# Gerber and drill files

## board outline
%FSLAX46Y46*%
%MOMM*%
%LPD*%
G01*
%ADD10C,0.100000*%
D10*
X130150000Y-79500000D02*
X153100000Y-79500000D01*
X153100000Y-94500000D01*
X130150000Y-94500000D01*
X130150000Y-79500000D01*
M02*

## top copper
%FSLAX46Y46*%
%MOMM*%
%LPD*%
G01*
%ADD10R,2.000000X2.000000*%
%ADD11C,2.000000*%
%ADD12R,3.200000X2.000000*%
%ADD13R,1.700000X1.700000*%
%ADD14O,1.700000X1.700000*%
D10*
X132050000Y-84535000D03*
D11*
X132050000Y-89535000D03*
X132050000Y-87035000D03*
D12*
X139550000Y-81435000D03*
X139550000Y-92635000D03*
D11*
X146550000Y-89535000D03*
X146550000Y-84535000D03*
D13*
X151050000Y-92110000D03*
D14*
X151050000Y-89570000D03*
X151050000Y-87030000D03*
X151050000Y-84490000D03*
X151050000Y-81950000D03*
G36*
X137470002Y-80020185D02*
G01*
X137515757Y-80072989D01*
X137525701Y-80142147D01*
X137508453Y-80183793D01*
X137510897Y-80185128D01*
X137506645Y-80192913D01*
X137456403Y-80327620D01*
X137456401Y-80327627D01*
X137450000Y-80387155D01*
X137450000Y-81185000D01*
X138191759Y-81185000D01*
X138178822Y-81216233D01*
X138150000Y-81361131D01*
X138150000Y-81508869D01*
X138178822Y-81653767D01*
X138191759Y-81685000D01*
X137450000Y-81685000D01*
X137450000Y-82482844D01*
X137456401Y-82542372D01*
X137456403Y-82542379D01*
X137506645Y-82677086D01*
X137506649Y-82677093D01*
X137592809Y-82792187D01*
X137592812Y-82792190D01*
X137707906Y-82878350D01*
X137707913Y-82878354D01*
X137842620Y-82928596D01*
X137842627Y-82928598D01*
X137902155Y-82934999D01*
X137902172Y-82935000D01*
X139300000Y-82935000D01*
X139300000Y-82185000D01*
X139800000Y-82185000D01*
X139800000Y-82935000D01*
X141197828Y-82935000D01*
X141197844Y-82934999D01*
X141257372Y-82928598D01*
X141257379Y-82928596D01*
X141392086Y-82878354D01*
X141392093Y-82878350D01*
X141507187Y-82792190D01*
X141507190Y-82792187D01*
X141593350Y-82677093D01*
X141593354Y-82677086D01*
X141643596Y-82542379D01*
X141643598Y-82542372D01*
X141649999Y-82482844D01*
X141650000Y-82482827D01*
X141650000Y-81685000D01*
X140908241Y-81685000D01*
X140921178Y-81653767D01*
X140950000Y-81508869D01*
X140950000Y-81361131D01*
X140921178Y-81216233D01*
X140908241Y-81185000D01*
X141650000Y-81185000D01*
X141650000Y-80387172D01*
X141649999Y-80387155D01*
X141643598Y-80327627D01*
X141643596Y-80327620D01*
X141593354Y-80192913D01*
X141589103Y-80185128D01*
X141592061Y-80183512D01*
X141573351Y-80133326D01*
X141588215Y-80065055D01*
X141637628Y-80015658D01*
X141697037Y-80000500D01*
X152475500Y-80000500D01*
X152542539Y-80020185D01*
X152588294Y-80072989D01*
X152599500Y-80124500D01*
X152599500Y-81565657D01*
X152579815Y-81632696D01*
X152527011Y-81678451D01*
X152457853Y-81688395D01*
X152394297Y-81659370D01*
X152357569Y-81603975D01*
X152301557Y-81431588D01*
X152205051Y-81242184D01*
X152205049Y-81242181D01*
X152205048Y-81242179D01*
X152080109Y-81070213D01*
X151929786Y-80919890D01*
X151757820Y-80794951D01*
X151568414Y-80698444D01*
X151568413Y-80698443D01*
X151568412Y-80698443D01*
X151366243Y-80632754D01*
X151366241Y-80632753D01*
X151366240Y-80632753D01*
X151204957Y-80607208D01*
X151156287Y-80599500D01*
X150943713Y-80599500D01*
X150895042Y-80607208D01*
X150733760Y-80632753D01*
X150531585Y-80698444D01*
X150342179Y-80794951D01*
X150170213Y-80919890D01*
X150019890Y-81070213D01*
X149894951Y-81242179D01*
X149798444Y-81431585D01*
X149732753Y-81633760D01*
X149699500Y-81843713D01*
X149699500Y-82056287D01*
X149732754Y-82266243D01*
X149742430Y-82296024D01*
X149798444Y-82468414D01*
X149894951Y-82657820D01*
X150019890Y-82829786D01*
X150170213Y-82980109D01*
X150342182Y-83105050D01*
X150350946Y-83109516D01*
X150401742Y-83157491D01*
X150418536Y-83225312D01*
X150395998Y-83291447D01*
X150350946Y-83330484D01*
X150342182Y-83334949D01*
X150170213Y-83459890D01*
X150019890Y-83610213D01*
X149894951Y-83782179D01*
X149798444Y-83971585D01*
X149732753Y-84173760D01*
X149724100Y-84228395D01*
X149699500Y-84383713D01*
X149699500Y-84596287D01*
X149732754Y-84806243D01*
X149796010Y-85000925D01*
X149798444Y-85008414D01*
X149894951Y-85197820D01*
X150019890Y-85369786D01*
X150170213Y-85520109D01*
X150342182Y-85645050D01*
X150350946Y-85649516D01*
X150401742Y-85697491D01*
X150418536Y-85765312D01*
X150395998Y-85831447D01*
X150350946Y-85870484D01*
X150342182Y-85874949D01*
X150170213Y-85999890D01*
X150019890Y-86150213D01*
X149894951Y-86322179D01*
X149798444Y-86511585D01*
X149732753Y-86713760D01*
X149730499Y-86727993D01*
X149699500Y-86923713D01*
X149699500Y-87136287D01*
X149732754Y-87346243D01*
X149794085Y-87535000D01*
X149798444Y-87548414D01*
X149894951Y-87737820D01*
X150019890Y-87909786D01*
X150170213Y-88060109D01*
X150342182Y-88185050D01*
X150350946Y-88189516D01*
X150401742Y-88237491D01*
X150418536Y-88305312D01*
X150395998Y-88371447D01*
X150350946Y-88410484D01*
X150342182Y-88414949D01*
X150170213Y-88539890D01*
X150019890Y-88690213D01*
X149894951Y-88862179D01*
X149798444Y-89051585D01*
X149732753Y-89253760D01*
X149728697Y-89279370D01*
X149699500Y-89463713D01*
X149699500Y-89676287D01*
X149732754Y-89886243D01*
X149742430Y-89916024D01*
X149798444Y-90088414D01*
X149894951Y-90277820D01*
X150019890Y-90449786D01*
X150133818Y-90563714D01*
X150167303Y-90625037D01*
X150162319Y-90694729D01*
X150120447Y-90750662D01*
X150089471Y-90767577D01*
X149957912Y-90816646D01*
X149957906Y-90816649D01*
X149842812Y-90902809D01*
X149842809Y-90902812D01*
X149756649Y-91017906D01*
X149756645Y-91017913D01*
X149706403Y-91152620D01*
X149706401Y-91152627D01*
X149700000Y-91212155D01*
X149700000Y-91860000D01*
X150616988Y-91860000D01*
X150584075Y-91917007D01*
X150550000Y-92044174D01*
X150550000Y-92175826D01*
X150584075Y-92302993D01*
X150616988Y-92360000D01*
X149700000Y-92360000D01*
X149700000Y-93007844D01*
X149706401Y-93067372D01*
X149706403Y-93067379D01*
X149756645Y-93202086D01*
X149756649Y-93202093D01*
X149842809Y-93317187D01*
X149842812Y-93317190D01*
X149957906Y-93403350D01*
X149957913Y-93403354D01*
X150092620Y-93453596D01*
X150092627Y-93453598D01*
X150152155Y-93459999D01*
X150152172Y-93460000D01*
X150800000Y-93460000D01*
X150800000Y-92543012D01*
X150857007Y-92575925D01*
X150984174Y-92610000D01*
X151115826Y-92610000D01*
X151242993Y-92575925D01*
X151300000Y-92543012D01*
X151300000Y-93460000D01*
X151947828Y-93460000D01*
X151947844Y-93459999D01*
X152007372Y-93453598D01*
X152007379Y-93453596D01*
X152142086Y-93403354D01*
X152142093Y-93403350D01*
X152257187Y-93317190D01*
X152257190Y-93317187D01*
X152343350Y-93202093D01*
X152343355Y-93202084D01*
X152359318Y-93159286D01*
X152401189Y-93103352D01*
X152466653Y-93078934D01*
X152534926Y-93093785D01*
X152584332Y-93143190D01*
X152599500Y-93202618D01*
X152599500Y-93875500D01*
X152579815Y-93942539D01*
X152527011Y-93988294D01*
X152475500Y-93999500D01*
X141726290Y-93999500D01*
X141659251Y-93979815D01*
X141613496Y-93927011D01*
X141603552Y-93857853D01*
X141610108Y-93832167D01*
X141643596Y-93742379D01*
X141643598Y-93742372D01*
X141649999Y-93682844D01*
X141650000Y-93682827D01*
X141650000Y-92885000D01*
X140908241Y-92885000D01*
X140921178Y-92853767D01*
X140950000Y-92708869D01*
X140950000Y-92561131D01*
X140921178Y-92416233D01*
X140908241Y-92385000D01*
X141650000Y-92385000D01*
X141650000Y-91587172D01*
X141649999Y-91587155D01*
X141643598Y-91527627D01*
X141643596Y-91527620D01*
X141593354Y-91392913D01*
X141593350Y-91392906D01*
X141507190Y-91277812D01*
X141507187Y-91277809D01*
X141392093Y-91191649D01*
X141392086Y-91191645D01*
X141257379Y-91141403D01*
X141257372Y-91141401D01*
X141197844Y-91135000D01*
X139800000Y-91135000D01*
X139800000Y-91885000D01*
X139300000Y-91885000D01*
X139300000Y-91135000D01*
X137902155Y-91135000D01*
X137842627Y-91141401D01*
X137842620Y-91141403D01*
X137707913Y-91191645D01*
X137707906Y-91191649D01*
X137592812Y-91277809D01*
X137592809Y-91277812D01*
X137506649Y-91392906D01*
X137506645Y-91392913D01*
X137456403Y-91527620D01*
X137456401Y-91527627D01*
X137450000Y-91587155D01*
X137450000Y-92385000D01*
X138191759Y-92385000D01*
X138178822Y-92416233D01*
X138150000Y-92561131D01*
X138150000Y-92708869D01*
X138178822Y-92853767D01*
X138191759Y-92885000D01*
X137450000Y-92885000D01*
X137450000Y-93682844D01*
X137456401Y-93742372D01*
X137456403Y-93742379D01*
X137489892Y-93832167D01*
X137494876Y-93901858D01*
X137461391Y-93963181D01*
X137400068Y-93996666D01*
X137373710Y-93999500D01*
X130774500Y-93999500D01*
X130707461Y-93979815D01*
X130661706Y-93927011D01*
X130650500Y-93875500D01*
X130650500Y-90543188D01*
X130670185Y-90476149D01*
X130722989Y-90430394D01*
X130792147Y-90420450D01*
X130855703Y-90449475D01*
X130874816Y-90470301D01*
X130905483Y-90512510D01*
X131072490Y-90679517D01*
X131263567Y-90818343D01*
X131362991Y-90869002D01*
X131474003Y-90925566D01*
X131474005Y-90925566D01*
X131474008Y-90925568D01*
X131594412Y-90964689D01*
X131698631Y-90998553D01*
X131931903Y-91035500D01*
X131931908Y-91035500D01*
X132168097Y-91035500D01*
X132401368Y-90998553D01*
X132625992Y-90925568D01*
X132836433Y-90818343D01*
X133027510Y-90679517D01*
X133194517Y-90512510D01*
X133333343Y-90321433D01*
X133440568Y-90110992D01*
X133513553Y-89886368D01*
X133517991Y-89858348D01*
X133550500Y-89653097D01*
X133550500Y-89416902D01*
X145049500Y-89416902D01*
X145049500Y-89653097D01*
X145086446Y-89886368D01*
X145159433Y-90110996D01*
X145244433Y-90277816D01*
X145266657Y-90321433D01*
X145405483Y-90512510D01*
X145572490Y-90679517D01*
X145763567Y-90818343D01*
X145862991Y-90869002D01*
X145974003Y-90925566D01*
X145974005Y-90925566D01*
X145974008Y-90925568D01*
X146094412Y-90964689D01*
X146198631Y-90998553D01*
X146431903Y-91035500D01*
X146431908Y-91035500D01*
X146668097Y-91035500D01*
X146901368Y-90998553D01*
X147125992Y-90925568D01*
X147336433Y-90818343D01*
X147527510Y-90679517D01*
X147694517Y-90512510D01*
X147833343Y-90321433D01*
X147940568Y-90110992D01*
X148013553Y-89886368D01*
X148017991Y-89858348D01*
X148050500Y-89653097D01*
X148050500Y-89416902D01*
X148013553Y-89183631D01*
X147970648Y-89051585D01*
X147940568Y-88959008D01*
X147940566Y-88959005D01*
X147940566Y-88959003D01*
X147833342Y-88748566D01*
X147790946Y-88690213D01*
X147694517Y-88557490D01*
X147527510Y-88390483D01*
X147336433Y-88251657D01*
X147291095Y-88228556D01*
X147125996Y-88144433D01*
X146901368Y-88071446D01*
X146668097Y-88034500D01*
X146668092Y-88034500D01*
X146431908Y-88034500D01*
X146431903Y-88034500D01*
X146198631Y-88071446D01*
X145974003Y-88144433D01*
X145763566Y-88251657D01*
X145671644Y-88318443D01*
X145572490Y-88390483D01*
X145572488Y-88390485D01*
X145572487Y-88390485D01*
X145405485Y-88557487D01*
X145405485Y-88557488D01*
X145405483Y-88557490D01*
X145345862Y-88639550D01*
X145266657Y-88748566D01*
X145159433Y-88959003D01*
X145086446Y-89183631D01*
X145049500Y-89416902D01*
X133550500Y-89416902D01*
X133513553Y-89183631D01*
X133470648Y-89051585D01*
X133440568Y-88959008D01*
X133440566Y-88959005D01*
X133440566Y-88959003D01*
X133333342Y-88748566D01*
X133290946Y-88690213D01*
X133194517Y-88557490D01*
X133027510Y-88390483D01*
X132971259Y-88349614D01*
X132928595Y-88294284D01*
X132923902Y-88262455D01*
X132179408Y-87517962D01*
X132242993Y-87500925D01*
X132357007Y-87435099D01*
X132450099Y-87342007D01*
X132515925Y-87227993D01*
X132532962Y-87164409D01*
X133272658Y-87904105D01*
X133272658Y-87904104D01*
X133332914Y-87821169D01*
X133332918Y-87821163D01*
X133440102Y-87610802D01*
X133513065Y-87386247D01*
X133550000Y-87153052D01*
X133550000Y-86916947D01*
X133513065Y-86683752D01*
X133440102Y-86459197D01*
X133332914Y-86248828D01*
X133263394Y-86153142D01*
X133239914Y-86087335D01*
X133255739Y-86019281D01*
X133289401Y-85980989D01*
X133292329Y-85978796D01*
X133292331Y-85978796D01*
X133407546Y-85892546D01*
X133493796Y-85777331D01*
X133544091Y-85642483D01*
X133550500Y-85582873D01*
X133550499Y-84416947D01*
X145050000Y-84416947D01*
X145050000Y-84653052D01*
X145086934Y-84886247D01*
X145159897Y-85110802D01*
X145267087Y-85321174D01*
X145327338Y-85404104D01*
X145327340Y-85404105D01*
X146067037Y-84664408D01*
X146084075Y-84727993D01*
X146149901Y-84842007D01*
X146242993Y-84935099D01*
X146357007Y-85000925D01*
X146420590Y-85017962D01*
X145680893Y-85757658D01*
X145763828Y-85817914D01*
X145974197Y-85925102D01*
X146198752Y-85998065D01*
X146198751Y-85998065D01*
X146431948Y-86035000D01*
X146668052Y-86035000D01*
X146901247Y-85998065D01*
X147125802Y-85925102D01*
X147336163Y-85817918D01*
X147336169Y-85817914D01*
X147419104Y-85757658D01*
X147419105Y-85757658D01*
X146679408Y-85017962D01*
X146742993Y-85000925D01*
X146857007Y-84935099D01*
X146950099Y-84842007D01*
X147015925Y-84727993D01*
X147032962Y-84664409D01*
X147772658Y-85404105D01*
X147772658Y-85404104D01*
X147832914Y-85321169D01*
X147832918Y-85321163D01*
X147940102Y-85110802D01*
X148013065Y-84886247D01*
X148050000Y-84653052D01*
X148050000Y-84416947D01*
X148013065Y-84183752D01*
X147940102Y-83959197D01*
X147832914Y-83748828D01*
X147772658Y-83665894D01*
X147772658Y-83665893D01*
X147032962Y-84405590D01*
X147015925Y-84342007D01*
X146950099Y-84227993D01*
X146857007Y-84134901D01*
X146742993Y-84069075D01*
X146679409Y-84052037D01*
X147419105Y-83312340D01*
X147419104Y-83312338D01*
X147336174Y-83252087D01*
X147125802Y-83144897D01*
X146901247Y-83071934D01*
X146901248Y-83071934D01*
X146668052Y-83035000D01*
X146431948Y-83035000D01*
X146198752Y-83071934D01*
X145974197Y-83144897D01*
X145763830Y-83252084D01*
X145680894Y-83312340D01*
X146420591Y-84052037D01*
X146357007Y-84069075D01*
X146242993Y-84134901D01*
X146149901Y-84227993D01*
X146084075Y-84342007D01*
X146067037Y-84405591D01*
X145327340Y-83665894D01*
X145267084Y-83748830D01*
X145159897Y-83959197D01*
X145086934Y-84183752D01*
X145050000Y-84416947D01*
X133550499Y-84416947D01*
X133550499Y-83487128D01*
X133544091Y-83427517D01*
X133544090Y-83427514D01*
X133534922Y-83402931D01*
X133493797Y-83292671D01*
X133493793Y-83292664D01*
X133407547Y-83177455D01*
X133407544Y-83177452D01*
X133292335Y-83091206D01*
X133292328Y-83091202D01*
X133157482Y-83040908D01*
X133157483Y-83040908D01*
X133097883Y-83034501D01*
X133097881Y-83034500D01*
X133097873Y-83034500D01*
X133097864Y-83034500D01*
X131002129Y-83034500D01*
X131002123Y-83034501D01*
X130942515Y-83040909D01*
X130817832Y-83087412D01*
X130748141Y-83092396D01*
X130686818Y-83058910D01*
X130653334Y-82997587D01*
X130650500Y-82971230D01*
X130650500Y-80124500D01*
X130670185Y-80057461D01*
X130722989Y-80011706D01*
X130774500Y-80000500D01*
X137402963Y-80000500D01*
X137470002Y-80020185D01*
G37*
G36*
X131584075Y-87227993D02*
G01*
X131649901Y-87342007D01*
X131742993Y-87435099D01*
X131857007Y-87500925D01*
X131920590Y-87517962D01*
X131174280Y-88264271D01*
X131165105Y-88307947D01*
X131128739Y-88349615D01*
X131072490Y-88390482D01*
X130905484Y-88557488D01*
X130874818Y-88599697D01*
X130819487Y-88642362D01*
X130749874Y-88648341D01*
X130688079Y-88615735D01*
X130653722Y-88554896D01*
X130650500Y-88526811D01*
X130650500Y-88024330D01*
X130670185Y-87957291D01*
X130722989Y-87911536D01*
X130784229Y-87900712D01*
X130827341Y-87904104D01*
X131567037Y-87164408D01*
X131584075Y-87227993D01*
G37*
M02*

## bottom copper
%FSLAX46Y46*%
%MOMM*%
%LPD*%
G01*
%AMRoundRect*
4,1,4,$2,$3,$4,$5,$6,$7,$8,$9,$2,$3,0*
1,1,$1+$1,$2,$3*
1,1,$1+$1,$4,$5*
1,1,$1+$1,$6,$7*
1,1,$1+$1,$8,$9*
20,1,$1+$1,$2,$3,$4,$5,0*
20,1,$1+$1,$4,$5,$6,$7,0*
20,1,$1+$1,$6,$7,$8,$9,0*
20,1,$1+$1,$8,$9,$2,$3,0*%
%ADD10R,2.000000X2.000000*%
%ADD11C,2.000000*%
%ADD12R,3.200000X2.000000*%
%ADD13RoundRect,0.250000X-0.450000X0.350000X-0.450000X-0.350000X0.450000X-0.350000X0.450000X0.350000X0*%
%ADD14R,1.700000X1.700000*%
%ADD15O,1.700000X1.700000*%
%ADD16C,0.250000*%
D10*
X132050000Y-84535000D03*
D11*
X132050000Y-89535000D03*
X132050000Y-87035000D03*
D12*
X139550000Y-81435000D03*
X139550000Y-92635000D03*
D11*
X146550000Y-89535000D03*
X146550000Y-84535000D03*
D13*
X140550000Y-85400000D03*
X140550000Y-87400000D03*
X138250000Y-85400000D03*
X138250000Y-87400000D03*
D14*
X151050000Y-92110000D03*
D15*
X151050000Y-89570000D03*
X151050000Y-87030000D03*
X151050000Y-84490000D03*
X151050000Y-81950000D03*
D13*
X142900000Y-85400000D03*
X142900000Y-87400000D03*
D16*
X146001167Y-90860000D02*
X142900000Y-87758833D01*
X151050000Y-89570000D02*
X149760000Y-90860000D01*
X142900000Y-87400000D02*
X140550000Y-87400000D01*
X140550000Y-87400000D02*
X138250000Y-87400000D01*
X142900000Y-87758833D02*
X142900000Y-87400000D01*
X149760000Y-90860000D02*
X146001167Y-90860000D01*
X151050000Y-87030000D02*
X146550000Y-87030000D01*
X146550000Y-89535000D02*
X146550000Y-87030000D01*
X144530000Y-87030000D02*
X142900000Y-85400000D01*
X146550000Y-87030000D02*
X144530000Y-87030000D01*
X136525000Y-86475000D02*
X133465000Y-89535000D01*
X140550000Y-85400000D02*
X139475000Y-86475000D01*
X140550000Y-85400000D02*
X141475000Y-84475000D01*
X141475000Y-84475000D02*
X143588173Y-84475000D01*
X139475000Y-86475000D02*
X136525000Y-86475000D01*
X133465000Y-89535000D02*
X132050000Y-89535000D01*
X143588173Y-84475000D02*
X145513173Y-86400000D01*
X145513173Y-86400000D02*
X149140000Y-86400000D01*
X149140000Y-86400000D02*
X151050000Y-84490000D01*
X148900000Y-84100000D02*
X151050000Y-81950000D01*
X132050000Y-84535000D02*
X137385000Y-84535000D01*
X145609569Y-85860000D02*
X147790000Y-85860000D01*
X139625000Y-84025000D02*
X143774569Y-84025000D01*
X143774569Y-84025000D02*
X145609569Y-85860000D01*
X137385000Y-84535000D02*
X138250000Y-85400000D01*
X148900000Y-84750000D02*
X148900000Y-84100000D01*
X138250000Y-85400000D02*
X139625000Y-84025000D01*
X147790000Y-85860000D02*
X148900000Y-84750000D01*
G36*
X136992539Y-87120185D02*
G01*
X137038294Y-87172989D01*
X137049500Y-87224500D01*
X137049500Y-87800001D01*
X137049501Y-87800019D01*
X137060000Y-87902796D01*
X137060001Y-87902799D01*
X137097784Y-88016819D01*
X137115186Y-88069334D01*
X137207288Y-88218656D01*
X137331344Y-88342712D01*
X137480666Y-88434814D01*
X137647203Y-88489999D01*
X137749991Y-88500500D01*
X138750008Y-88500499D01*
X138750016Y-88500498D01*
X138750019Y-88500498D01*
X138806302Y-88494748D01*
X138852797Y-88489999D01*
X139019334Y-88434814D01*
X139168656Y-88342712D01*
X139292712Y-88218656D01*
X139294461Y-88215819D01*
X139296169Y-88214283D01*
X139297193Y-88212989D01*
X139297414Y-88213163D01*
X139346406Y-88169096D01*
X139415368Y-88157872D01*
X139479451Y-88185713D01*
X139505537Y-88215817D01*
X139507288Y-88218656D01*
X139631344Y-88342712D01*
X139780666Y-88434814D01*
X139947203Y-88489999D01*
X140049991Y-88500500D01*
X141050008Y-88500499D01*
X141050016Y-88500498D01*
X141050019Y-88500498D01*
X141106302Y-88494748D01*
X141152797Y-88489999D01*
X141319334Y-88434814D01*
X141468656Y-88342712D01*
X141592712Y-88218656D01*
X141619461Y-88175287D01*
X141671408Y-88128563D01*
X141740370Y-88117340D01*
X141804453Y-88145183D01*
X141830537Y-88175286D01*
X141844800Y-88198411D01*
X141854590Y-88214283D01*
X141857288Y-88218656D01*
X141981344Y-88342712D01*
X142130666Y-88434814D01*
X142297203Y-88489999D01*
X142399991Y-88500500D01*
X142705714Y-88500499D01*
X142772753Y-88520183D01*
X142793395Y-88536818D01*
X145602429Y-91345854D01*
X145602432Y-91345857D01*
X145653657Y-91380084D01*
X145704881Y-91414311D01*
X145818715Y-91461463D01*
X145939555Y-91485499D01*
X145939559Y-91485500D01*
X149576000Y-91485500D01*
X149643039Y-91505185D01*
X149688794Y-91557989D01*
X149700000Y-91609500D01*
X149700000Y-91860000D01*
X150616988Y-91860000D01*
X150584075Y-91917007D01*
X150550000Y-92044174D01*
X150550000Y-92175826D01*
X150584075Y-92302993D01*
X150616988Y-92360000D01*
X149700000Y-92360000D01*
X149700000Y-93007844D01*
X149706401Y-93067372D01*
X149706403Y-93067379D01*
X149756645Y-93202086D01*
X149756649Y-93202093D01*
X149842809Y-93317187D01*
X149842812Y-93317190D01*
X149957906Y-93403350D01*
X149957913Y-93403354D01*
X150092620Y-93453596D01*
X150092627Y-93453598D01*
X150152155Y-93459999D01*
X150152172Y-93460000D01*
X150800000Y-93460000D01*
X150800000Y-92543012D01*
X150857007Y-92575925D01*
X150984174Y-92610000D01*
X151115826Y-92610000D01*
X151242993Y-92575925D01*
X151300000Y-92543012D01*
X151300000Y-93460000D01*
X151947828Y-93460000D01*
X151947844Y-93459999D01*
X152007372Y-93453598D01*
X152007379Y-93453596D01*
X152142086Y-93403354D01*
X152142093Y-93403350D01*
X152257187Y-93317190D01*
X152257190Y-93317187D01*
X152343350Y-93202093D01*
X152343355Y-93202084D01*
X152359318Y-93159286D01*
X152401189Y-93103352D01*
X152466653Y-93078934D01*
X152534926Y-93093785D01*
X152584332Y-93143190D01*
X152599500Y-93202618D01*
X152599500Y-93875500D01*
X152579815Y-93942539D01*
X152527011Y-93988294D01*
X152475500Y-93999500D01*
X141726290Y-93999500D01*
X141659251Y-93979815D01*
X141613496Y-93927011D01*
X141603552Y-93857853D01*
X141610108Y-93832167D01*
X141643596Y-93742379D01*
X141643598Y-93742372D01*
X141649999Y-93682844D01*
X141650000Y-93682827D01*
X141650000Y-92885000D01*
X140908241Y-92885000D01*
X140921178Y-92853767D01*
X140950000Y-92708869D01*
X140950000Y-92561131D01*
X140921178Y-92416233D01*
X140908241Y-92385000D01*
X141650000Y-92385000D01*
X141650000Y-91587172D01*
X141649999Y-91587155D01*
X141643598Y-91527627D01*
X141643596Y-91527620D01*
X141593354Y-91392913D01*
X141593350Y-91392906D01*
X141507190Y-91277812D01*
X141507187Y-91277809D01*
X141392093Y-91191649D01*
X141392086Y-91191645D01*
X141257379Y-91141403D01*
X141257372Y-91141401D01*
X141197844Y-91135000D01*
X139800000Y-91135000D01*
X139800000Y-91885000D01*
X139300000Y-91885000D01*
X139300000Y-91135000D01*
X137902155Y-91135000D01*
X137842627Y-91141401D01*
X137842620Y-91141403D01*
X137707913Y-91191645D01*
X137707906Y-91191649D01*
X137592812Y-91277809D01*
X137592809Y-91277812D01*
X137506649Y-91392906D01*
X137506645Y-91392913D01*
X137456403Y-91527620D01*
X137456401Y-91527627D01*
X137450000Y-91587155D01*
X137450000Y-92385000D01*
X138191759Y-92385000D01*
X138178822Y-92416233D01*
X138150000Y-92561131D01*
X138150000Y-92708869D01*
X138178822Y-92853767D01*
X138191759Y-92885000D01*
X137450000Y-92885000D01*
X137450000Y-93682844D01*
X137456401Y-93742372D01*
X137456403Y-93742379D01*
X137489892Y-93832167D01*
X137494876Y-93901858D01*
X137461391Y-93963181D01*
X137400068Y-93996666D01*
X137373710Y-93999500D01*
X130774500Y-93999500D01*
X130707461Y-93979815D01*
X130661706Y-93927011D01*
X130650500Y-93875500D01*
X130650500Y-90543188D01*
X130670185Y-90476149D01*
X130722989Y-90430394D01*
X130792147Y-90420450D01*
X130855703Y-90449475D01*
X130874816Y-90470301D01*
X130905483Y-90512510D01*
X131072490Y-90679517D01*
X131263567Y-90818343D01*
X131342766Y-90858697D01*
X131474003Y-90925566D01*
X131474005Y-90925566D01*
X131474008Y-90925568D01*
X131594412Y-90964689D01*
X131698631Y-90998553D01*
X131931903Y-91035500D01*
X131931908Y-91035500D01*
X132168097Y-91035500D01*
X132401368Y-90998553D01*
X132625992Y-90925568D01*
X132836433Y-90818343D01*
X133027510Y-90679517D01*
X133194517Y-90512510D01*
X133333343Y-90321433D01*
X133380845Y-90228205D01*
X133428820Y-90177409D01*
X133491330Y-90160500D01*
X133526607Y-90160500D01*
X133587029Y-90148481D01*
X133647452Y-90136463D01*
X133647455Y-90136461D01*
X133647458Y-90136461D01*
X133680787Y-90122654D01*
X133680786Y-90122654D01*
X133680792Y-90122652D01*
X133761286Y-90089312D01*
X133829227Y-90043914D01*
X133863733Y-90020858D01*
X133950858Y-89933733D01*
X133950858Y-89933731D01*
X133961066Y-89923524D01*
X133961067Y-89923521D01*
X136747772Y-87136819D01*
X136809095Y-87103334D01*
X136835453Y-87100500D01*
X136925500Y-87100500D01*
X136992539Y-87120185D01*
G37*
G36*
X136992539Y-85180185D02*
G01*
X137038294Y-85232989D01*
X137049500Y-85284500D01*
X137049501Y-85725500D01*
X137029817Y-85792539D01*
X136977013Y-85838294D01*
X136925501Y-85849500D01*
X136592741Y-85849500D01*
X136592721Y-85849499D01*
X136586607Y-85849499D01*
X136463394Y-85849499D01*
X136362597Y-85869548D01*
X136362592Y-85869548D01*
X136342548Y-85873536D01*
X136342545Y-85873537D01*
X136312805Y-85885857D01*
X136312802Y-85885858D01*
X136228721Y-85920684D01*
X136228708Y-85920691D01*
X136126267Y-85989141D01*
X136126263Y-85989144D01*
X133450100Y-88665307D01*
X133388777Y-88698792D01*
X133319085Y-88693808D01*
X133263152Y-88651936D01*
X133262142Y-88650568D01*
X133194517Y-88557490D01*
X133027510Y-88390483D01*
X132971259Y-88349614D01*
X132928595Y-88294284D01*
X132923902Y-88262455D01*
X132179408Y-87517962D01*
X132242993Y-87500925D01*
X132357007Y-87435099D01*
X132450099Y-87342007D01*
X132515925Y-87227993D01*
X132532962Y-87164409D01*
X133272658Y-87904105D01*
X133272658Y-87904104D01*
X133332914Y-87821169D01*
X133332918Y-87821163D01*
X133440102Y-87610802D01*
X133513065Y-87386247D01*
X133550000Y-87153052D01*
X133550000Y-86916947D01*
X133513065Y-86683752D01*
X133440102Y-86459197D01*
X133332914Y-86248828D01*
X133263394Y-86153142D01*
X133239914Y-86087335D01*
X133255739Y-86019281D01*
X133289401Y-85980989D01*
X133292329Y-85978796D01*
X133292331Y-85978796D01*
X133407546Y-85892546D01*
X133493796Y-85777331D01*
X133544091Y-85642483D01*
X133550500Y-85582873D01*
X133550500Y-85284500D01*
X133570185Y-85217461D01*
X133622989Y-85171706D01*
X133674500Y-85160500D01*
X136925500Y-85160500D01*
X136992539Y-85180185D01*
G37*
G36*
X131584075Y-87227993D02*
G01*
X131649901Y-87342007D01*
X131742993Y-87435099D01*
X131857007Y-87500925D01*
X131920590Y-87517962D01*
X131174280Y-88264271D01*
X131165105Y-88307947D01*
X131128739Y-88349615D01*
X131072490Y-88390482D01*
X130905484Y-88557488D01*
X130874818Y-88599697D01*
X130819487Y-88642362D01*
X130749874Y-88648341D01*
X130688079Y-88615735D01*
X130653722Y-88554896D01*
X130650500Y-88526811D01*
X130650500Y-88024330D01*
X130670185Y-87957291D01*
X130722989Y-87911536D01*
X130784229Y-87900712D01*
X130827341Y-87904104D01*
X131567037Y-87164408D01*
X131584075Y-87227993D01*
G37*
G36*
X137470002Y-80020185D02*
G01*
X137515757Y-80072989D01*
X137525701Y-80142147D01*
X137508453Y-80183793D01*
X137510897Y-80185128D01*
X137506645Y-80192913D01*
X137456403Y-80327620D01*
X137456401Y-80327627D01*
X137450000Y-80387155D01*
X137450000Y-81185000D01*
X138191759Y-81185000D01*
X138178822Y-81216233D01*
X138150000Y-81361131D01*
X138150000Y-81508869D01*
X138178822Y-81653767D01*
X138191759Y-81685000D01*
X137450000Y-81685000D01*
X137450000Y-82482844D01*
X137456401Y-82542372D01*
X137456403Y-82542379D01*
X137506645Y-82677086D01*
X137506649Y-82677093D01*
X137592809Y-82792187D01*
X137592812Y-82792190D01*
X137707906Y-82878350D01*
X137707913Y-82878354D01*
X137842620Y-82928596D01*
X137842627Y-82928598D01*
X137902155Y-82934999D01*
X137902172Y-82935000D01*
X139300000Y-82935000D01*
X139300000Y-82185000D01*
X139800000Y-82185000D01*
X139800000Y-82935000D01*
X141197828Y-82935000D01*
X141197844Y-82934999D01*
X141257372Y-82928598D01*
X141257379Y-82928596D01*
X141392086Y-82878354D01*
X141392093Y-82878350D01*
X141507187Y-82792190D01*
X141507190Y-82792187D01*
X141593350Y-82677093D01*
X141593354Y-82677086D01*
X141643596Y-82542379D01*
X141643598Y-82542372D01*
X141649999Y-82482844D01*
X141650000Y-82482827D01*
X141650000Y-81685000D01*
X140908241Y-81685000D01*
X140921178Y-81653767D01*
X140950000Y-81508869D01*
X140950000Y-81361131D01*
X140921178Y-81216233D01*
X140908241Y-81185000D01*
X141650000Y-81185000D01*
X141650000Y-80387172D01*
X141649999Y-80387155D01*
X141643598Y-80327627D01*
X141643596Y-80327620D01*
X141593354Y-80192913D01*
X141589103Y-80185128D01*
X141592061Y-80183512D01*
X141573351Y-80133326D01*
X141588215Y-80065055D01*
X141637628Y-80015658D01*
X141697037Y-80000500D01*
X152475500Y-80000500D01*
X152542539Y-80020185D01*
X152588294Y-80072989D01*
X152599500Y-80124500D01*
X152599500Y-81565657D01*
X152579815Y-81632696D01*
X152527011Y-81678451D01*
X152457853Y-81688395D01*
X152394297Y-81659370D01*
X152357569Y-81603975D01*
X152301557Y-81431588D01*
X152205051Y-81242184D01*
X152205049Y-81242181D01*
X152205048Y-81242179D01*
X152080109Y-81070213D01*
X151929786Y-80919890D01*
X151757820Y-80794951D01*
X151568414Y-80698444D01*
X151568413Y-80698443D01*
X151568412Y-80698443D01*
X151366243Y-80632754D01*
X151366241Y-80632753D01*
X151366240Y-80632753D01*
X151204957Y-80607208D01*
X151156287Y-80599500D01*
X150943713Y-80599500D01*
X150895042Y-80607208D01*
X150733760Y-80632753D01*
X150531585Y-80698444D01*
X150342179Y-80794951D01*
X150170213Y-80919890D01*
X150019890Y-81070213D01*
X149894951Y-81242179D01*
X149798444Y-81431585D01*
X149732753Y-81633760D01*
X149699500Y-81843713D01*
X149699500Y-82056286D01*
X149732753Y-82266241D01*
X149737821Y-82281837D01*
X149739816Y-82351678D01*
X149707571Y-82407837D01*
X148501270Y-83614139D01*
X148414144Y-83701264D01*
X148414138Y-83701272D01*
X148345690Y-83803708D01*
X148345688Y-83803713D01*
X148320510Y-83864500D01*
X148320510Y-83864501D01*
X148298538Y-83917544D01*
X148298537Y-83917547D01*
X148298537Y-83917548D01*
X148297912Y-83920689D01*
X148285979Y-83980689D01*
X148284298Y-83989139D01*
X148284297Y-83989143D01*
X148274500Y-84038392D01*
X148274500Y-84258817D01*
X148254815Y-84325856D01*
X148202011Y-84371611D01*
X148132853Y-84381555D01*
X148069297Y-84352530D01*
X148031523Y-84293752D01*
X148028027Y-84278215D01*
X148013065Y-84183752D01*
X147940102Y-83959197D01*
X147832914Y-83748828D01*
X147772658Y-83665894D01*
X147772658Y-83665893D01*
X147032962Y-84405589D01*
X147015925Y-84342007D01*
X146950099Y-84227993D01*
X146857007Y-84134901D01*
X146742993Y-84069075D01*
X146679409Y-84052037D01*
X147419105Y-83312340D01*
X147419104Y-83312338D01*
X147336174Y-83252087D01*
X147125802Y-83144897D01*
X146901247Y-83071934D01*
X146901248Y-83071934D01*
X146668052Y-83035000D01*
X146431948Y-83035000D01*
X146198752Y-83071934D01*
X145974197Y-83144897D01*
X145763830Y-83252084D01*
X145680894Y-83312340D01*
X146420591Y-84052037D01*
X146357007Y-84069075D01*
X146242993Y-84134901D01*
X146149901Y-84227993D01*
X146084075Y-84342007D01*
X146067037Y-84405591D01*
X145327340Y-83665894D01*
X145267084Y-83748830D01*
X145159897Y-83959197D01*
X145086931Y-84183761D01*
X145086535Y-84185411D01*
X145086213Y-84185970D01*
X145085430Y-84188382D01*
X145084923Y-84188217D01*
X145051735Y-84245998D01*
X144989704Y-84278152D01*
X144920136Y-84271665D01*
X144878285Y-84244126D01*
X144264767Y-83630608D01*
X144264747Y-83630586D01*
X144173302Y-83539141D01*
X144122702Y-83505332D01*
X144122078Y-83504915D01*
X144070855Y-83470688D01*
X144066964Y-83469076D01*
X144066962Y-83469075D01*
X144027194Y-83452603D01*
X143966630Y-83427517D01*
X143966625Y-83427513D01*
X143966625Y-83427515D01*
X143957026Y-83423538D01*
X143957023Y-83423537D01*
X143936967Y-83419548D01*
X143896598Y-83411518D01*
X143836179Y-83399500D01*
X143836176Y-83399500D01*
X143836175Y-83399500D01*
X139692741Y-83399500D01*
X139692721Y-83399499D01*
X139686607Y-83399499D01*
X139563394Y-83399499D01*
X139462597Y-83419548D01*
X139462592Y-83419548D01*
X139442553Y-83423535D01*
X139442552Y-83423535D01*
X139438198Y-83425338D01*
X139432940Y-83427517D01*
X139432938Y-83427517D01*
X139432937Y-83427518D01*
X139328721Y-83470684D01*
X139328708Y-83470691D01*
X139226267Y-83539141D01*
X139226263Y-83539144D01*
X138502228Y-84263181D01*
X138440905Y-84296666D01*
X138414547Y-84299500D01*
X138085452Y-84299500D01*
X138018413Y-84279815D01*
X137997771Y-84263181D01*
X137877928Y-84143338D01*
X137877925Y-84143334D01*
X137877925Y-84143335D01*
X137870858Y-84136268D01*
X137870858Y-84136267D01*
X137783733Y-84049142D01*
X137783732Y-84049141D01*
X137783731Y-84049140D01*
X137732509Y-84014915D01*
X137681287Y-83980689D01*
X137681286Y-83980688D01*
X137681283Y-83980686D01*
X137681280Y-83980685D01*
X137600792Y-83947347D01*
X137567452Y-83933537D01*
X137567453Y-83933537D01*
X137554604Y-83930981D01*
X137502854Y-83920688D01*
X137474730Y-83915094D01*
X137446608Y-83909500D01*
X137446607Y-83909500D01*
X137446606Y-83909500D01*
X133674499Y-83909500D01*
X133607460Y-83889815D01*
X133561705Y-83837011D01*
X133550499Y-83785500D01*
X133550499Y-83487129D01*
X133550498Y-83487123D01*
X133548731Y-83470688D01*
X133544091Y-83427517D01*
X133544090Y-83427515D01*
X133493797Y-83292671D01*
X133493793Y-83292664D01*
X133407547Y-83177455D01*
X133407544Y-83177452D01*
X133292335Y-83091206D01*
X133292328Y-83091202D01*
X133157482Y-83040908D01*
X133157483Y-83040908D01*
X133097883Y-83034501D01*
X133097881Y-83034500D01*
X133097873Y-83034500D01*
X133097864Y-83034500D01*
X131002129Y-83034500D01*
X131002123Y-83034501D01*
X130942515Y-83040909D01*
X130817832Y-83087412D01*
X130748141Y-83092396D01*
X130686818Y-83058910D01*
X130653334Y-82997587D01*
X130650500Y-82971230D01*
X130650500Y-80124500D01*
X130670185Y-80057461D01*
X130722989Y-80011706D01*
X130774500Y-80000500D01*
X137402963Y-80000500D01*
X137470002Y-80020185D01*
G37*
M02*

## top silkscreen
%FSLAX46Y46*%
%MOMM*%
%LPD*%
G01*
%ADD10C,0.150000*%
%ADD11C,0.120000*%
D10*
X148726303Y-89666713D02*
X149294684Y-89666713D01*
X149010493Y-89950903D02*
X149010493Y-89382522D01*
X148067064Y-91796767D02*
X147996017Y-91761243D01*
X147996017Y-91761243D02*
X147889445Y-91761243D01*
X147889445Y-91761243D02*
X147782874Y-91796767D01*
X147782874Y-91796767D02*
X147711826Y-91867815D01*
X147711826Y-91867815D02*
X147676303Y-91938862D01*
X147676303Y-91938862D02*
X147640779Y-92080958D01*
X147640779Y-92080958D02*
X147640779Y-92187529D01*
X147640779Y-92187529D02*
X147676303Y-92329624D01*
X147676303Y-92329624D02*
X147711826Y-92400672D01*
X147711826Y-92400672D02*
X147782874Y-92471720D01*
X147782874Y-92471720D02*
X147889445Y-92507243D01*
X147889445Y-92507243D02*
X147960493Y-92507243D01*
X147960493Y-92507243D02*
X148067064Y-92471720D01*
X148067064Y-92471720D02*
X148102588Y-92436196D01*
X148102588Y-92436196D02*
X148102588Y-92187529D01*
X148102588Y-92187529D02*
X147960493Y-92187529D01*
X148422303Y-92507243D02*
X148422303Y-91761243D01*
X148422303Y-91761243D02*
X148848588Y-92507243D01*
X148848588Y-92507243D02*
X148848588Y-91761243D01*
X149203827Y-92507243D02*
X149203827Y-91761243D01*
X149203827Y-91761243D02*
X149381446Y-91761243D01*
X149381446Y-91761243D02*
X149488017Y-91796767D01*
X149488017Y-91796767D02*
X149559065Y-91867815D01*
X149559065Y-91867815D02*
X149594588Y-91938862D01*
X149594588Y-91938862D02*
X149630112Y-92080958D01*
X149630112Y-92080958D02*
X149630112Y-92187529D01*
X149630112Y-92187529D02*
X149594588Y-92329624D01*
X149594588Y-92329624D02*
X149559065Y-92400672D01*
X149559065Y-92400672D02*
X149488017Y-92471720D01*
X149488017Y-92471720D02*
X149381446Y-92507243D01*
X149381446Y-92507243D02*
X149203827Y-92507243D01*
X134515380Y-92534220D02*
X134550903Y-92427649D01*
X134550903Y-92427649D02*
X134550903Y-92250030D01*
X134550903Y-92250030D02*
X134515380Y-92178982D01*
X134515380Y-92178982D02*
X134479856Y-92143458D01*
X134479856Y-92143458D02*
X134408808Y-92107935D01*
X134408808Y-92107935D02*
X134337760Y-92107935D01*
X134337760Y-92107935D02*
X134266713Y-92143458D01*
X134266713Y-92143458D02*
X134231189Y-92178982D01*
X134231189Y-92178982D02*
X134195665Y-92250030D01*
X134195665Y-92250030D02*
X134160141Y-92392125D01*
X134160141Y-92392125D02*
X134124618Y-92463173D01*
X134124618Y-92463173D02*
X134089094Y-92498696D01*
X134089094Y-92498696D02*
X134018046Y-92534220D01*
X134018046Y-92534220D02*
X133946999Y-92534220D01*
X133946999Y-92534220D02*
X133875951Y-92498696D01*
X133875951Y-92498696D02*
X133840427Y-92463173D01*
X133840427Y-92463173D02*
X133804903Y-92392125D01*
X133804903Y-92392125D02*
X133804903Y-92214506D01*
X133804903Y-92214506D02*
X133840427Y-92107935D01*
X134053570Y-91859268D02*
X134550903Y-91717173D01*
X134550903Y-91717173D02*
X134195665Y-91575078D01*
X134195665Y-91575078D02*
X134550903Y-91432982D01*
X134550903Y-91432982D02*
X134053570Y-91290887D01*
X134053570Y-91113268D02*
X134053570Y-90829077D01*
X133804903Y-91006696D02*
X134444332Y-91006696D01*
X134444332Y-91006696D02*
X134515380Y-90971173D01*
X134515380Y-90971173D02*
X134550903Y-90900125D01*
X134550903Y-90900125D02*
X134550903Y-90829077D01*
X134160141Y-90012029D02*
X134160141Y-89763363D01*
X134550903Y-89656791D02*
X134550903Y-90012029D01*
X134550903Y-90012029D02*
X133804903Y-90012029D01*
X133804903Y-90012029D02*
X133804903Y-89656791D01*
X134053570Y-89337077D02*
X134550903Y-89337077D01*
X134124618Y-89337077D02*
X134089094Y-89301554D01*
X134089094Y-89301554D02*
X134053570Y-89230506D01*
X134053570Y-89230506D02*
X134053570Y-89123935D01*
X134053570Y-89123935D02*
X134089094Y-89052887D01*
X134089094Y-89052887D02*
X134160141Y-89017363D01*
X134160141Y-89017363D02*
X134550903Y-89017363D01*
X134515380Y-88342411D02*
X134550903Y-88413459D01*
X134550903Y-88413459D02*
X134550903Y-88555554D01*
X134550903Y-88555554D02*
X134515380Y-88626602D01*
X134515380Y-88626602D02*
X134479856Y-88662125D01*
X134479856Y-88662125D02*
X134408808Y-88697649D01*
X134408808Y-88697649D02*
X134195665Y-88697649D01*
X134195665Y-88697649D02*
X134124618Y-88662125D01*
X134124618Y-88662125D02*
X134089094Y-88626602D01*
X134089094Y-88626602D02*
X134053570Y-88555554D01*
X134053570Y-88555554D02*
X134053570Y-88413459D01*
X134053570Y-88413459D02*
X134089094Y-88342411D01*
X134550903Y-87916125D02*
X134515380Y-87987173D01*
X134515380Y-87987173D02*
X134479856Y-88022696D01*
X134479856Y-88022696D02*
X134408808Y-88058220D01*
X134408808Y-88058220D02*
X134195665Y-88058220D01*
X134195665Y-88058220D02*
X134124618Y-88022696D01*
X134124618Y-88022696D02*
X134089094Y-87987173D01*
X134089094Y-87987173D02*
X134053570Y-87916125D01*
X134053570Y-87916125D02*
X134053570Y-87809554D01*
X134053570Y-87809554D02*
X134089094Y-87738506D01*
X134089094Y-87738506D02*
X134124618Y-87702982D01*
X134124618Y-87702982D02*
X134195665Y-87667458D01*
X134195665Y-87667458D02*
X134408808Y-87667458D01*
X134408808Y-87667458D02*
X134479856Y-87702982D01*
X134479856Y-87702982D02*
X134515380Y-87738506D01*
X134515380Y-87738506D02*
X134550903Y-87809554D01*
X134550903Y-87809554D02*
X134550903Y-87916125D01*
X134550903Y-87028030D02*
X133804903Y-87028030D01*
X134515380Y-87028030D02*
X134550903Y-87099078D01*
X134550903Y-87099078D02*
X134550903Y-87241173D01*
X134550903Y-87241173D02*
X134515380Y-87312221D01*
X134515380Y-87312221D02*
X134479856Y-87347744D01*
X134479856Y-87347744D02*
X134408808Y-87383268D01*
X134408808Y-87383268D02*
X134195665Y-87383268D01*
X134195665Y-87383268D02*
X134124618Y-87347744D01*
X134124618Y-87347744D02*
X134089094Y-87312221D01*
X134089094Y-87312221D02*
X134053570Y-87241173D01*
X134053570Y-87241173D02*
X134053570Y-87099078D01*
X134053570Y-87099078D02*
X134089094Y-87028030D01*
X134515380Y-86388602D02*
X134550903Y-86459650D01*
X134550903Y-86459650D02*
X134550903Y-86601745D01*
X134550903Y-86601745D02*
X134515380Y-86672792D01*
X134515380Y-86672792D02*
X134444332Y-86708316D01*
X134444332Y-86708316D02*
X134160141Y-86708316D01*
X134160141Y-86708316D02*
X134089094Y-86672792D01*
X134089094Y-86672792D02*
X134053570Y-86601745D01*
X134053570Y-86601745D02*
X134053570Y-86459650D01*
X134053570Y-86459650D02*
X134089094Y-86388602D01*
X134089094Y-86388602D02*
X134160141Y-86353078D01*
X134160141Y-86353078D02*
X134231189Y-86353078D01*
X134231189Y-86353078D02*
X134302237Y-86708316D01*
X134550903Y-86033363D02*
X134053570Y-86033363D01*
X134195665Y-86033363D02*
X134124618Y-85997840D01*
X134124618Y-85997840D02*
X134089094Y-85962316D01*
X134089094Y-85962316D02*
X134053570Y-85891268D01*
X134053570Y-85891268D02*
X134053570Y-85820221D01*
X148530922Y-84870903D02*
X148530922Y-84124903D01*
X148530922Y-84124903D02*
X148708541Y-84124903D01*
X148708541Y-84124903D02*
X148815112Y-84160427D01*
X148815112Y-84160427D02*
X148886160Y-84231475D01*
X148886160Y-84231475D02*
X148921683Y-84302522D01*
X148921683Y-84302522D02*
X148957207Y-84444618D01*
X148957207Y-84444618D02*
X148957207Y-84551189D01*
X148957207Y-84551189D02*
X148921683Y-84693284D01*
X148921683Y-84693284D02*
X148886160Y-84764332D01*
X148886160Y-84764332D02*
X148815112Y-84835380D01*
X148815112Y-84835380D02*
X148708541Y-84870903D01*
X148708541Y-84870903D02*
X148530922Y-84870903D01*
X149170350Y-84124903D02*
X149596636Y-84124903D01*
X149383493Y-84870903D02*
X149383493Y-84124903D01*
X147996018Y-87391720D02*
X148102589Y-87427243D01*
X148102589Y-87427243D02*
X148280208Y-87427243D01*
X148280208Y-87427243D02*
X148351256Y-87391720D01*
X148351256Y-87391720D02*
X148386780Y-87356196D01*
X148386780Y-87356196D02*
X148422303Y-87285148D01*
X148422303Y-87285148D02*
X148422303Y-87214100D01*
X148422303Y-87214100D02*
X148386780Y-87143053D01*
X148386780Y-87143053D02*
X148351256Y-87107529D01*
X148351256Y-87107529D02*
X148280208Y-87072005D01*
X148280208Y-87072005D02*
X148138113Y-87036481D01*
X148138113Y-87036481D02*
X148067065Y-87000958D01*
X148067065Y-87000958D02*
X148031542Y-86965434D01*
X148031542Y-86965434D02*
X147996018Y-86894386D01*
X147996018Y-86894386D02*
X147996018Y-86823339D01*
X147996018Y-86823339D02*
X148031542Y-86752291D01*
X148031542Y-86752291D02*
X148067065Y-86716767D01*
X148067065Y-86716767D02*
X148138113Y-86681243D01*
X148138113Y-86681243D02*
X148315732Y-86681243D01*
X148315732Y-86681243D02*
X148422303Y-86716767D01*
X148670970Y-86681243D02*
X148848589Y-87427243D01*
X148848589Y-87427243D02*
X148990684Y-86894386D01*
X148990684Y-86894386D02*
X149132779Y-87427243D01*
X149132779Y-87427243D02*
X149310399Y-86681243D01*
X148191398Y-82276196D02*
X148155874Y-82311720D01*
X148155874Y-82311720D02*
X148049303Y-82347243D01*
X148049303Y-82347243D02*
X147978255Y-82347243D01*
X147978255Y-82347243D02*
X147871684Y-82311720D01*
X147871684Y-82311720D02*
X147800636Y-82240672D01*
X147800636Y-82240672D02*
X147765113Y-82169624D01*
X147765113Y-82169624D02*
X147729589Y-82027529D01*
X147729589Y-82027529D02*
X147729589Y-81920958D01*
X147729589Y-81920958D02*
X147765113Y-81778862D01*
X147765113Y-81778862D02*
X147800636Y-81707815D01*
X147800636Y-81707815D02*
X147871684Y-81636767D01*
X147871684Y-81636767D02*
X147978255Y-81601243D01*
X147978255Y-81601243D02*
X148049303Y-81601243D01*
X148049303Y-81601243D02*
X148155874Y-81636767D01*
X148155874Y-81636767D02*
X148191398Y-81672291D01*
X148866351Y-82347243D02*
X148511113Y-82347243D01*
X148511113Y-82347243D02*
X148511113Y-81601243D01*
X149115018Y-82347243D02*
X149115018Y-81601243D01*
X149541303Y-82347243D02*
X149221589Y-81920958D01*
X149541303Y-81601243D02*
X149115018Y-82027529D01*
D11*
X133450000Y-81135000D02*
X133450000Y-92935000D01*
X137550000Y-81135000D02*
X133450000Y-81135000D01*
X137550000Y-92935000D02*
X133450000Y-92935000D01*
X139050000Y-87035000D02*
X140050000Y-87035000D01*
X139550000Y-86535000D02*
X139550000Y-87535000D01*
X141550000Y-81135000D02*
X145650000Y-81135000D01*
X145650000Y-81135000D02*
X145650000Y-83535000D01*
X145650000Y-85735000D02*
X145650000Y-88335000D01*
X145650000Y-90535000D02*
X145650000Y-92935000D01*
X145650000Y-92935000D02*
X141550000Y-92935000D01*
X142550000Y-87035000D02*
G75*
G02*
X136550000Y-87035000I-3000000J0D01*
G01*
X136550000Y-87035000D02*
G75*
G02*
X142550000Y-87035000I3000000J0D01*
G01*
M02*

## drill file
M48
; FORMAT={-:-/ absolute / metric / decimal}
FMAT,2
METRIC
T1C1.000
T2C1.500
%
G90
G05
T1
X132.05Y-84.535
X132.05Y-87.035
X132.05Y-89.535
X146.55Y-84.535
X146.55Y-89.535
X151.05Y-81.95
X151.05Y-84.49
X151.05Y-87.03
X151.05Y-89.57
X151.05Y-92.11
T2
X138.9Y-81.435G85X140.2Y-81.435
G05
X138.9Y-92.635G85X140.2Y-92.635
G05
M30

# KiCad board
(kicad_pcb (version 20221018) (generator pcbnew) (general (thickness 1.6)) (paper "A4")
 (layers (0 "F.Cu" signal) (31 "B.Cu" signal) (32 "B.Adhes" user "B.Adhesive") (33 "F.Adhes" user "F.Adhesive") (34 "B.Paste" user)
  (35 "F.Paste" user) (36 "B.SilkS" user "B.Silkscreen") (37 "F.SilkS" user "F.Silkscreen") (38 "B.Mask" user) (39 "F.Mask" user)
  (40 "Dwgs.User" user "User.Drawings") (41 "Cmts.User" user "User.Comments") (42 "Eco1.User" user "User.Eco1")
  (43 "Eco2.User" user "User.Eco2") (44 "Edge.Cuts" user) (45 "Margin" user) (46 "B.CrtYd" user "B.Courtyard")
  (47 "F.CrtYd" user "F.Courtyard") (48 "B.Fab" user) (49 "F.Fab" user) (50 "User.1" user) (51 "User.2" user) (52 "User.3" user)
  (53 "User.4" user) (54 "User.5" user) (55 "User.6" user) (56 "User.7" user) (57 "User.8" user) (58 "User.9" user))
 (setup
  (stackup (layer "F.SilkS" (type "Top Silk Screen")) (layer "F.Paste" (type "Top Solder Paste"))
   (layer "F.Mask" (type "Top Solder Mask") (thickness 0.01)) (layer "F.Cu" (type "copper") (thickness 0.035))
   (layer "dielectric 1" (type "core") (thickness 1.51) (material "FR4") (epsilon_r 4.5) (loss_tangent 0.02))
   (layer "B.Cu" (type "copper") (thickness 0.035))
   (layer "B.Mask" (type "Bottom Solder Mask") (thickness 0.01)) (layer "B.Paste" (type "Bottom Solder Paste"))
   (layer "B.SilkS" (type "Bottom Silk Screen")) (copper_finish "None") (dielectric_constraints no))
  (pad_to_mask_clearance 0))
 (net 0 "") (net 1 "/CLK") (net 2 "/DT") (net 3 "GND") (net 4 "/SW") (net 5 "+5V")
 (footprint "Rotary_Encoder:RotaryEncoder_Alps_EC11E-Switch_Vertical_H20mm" (layer "F.Cu") (at 132.05 84.535)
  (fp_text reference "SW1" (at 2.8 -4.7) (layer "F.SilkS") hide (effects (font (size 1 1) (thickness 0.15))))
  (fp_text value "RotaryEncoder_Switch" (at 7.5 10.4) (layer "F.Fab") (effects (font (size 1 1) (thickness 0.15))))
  (fp_line (start 1.4 -3.4) (end 1.4 8.4) (stroke (width 0.12) (type solid)) (layer "F.SilkS"))
  (fp_line (start 5.5 -3.4) (end 1.4 -3.4) (stroke (width 0.12) (type solid)) (layer "F.SilkS"))
  (fp_line (start 5.5 8.4) (end 1.4 8.4) (stroke (width 0.12) (type solid)) (layer "F.SilkS"))
  (fp_line (start 7 2.5) (end 8 2.5) (stroke (width 0.12) (type solid)) (layer "F.SilkS"))
  (fp_line (start 7.5 2) (end 7.5 3) (stroke (width 0.12) (type solid)) (layer "F.SilkS"))
  (fp_line (start 9.5 -3.4) (end 13.6 -3.4) (stroke (width 0.12) (type solid)) (layer "F.SilkS"))
  (fp_line (start 13.6 -3.4) (end 13.6 -1) (stroke (width 0.12) (type solid)) (layer "F.SilkS"))
  (fp_line (start 13.6 1.2) (end 13.6 3.8) (stroke (width 0.12) (type solid)) (layer "F.SilkS"))
  (fp_line (start 13.6 6) (end 13.6 8.4) (stroke (width 0.12) (type solid)) (layer "F.SilkS"))
  (fp_line (start 13.6 8.4) (end 9.5 8.4) (stroke (width 0.12) (type solid)) (layer "F.SilkS"))
  (fp_circle (center 7.5 2.5) (end 10.5 2.5) (stroke (width 0.12) (type solid)) (fill none) (layer "F.SilkS"))
  (pad "A" thru_hole rect (at 0 0) (size 2 2) (drill 1) (layers "*.Cu" "*.Mask") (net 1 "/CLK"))
  (pad "B" thru_hole circle (at 0 5) (size 2 2) (drill 1) (layers "*.Cu" "*.Mask") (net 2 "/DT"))
  (pad "C" thru_hole circle (at 0 2.5) (size 2 2) (drill 1) (layers "*.Cu" "*.Mask") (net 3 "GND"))
  (pad "MP" thru_hole rect (at 7.5 -3.1) (size 3.2 2) (drill oval 2.8 1.5) (layers "*.Cu" "*.Mask") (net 3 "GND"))
  (pad "MP" thru_hole rect (at 7.5 8.1) (size 3.2 2) (drill oval 2.8 1.5) (layers "*.Cu" "*.Mask") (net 3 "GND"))
  (pad "S1" thru_hole circle (at 14.5 5) (size 2 2) (drill 1) (layers "*.Cu" "*.Mask") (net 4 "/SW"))
  (pad "S2" thru_hole circle (at 14.5 0) (size 2 2) (drill 1) (layers "*.Cu" "*.Mask") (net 3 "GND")))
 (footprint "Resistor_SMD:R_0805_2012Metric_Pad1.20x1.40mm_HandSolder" (layer "B.Cu") (at 140.55 86.4 -90)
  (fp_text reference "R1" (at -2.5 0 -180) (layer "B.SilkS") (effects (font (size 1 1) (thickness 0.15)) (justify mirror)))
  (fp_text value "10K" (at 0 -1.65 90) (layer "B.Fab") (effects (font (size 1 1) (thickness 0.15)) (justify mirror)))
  (pad "1" smd roundrect (at -1 0 270) (size 1.2 1.4) (layers "B.Cu" "B.Paste" "B.Mask") (roundrect_rratio 0.208333) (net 2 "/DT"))
  (pad "2" smd roundrect (at 1 0 270) (size 1.2 1.4) (layers "B.Cu" "B.Paste" "B.Mask") (roundrect_rratio 0.208333) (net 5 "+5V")))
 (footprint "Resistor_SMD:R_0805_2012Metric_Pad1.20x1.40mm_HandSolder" (layer "B.Cu") (at 138.25 86.4 -90)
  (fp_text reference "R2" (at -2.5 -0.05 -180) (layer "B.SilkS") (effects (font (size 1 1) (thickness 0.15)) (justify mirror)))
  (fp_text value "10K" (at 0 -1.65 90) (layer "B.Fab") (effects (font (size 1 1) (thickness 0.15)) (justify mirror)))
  (pad "1" smd roundrect (at -1 0 270) (size 1.2 1.4) (layers "B.Cu" "B.Paste" "B.Mask") (roundrect_rratio 0.208333) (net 1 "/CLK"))
  (pad "2" smd roundrect (at 1 0 270) (size 1.2 1.4) (layers "B.Cu" "B.Paste" "B.Mask") (roundrect_rratio 0.208333) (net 5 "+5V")))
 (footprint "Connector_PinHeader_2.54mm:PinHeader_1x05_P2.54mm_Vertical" (layer "B.Cu") (at 151.05 92.11)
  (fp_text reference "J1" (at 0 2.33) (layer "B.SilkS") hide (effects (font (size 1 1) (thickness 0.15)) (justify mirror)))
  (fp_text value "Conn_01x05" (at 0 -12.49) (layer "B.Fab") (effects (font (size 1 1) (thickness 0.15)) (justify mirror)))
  (pad "1" thru_hole rect (at 0 0) (size 1.7 1.7) (drill 1) (layers "*.Cu" "*.Mask") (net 3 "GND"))
  (pad "2" thru_hole oval (at 0 -2.54) (size 1.7 1.7) (drill 1) (layers "*.Cu" "*.Mask") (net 5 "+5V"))
  (pad "3" thru_hole oval (at 0 -5.08) (size 1.7 1.7) (drill 1) (layers "*.Cu" "*.Mask") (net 4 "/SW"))
  (pad "4" thru_hole oval (at 0 -7.62) (size 1.7 1.7) (drill 1) (layers "*.Cu" "*.Mask") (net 2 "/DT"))
  (pad "5" thru_hole oval (at 0 -10.16) (size 1.7 1.7) (drill 1) (layers "*.Cu" "*.Mask") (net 1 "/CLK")))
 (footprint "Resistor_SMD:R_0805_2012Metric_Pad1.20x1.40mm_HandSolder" (layer "B.Cu") (at 142.9 86.4 -90)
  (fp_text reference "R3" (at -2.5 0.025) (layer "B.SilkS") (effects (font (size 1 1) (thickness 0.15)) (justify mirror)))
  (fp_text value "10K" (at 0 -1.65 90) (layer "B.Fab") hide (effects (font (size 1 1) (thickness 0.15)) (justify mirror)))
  (pad "1" smd roundrect (at -1 0 270) (size 1.2 1.4) (layers "B.Cu" "B.Paste" "B.Mask") (roundrect_rratio 0.208333) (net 4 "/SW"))
  (pad "2" smd roundrect (at 1 0 270) (size 1.2 1.4) (layers "B.Cu" "B.Paste" "B.Mask") (roundrect_rratio 0.208333) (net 5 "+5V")))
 (gr_rect (start 130.15 79.5) (end 153.1 94.5) (stroke (width 0.1) (type default)) (fill none) (layer "Edge.Cuts"))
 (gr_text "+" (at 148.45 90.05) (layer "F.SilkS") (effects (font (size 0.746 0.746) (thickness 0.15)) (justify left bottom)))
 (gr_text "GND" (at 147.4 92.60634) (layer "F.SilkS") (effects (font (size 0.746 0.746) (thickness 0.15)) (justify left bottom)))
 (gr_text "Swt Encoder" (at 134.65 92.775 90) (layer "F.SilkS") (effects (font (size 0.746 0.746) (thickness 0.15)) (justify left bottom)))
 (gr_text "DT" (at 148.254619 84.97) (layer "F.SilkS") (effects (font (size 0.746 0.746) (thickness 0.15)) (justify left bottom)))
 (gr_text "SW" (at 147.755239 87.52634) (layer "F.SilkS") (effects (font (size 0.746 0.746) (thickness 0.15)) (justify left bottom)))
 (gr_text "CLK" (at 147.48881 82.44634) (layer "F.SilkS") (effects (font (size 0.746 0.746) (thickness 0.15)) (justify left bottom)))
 (segment (start 146.001167 90.86) (end 142.9 87.758833) (width 0.25) (layer "B.Cu") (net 5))
 (segment (start 151.05 89.57) (end 149.76 90.86) (width 0.25) (layer "B.Cu") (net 5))
 (segment (start 142.9 87.4) (end 140.55 87.4) (width 0.25) (layer "B.Cu") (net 5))
 (segment (start 140.55 87.4) (end 138.25 87.4) (width 0.25) (layer "B.Cu") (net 5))
 (segment (start 142.9 87.758833) (end 142.9 87.4) (width 0.25) (layer "B.Cu") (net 5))
 (segment (start 149.76 90.86) (end 146.001167 90.86) (width 0.25) (layer "B.Cu") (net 5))
 (segment (start 151.05 87.03) (end 146.55 87.03) (width 0.25) (layer "B.Cu") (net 4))
 (segment (start 146.55 89.535) (end 146.55 87.03) (width 0.25) (layer "B.Cu") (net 4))
 (segment (start 144.53 87.03) (end 142.9 85.4) (width 0.25) (layer "B.Cu") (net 4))
 (segment (start 146.55 87.03) (end 144.53 87.03) (width 0.25) (layer "B.Cu") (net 4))
 (segment (start 136.525 86.475) (end 133.465 89.535) (width 0.25) (layer "B.Cu") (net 2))
 (segment (start 140.55 85.4) (end 139.475 86.475) (width 0.25) (layer "B.Cu") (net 2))
 (segment (start 140.55 85.4) (end 141.475 84.475) (width 0.25) (layer "B.Cu") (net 2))
 (segment (start 141.475 84.475) (end 143.588173 84.475) (width 0.25) (layer "B.Cu") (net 2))
 (segment (start 139.475 86.475) (end 136.525 86.475) (width 0.25) (layer "B.Cu") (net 2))
 (segment (start 133.465 89.535) (end 132.05 89.535) (width 0.25) (layer "B.Cu") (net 2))
 (segment (start 143.588173 84.475) (end 145.513173 86.4) (width 0.25) (layer "B.Cu") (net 2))
 (segment (start 145.513173 86.4) (end 149.14 86.4) (width 0.25) (layer "B.Cu") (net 2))
 (segment (start 149.14 86.4) (end 151.05 84.49) (width 0.25) (layer "B.Cu") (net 2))
 (segment (start 148.9 84.1) (end 151.05 81.95) (width 0.25) (layer "B.Cu") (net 1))
 (segment (start 132.05 84.535) (end 137.385 84.535) (width 0.25) (layer "B.Cu") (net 1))
 (segment (start 145.609569 85.86) (end 147.79 85.86) (width 0.25) (layer "B.Cu") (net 1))
 (segment (start 139.625 84.025) (end 143.774569 84.025) (width 0.25) (layer "B.Cu") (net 1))
 (segment (start 143.774569 84.025) (end 145.609569 85.86) (width 0.25) (layer "B.Cu") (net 1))
 (segment (start 137.385 84.535) (end 138.25 85.4) (width 0.25) (layer "B.Cu") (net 1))
 (segment (start 148.9 84.75) (end 148.9 84.1) (width 0.25) (layer "B.Cu") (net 1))
 (segment (start 138.25 85.4) (end 139.625 84.025) (width 0.25) (layer "B.Cu") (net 1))
 (segment (start 147.79 85.86) (end 148.9 84.75) (width 0.25) (layer "B.Cu") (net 1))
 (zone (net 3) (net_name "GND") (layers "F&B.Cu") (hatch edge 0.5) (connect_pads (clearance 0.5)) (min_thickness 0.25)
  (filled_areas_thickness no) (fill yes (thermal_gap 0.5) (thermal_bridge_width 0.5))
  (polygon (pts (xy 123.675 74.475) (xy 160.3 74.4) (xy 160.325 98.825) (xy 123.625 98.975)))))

